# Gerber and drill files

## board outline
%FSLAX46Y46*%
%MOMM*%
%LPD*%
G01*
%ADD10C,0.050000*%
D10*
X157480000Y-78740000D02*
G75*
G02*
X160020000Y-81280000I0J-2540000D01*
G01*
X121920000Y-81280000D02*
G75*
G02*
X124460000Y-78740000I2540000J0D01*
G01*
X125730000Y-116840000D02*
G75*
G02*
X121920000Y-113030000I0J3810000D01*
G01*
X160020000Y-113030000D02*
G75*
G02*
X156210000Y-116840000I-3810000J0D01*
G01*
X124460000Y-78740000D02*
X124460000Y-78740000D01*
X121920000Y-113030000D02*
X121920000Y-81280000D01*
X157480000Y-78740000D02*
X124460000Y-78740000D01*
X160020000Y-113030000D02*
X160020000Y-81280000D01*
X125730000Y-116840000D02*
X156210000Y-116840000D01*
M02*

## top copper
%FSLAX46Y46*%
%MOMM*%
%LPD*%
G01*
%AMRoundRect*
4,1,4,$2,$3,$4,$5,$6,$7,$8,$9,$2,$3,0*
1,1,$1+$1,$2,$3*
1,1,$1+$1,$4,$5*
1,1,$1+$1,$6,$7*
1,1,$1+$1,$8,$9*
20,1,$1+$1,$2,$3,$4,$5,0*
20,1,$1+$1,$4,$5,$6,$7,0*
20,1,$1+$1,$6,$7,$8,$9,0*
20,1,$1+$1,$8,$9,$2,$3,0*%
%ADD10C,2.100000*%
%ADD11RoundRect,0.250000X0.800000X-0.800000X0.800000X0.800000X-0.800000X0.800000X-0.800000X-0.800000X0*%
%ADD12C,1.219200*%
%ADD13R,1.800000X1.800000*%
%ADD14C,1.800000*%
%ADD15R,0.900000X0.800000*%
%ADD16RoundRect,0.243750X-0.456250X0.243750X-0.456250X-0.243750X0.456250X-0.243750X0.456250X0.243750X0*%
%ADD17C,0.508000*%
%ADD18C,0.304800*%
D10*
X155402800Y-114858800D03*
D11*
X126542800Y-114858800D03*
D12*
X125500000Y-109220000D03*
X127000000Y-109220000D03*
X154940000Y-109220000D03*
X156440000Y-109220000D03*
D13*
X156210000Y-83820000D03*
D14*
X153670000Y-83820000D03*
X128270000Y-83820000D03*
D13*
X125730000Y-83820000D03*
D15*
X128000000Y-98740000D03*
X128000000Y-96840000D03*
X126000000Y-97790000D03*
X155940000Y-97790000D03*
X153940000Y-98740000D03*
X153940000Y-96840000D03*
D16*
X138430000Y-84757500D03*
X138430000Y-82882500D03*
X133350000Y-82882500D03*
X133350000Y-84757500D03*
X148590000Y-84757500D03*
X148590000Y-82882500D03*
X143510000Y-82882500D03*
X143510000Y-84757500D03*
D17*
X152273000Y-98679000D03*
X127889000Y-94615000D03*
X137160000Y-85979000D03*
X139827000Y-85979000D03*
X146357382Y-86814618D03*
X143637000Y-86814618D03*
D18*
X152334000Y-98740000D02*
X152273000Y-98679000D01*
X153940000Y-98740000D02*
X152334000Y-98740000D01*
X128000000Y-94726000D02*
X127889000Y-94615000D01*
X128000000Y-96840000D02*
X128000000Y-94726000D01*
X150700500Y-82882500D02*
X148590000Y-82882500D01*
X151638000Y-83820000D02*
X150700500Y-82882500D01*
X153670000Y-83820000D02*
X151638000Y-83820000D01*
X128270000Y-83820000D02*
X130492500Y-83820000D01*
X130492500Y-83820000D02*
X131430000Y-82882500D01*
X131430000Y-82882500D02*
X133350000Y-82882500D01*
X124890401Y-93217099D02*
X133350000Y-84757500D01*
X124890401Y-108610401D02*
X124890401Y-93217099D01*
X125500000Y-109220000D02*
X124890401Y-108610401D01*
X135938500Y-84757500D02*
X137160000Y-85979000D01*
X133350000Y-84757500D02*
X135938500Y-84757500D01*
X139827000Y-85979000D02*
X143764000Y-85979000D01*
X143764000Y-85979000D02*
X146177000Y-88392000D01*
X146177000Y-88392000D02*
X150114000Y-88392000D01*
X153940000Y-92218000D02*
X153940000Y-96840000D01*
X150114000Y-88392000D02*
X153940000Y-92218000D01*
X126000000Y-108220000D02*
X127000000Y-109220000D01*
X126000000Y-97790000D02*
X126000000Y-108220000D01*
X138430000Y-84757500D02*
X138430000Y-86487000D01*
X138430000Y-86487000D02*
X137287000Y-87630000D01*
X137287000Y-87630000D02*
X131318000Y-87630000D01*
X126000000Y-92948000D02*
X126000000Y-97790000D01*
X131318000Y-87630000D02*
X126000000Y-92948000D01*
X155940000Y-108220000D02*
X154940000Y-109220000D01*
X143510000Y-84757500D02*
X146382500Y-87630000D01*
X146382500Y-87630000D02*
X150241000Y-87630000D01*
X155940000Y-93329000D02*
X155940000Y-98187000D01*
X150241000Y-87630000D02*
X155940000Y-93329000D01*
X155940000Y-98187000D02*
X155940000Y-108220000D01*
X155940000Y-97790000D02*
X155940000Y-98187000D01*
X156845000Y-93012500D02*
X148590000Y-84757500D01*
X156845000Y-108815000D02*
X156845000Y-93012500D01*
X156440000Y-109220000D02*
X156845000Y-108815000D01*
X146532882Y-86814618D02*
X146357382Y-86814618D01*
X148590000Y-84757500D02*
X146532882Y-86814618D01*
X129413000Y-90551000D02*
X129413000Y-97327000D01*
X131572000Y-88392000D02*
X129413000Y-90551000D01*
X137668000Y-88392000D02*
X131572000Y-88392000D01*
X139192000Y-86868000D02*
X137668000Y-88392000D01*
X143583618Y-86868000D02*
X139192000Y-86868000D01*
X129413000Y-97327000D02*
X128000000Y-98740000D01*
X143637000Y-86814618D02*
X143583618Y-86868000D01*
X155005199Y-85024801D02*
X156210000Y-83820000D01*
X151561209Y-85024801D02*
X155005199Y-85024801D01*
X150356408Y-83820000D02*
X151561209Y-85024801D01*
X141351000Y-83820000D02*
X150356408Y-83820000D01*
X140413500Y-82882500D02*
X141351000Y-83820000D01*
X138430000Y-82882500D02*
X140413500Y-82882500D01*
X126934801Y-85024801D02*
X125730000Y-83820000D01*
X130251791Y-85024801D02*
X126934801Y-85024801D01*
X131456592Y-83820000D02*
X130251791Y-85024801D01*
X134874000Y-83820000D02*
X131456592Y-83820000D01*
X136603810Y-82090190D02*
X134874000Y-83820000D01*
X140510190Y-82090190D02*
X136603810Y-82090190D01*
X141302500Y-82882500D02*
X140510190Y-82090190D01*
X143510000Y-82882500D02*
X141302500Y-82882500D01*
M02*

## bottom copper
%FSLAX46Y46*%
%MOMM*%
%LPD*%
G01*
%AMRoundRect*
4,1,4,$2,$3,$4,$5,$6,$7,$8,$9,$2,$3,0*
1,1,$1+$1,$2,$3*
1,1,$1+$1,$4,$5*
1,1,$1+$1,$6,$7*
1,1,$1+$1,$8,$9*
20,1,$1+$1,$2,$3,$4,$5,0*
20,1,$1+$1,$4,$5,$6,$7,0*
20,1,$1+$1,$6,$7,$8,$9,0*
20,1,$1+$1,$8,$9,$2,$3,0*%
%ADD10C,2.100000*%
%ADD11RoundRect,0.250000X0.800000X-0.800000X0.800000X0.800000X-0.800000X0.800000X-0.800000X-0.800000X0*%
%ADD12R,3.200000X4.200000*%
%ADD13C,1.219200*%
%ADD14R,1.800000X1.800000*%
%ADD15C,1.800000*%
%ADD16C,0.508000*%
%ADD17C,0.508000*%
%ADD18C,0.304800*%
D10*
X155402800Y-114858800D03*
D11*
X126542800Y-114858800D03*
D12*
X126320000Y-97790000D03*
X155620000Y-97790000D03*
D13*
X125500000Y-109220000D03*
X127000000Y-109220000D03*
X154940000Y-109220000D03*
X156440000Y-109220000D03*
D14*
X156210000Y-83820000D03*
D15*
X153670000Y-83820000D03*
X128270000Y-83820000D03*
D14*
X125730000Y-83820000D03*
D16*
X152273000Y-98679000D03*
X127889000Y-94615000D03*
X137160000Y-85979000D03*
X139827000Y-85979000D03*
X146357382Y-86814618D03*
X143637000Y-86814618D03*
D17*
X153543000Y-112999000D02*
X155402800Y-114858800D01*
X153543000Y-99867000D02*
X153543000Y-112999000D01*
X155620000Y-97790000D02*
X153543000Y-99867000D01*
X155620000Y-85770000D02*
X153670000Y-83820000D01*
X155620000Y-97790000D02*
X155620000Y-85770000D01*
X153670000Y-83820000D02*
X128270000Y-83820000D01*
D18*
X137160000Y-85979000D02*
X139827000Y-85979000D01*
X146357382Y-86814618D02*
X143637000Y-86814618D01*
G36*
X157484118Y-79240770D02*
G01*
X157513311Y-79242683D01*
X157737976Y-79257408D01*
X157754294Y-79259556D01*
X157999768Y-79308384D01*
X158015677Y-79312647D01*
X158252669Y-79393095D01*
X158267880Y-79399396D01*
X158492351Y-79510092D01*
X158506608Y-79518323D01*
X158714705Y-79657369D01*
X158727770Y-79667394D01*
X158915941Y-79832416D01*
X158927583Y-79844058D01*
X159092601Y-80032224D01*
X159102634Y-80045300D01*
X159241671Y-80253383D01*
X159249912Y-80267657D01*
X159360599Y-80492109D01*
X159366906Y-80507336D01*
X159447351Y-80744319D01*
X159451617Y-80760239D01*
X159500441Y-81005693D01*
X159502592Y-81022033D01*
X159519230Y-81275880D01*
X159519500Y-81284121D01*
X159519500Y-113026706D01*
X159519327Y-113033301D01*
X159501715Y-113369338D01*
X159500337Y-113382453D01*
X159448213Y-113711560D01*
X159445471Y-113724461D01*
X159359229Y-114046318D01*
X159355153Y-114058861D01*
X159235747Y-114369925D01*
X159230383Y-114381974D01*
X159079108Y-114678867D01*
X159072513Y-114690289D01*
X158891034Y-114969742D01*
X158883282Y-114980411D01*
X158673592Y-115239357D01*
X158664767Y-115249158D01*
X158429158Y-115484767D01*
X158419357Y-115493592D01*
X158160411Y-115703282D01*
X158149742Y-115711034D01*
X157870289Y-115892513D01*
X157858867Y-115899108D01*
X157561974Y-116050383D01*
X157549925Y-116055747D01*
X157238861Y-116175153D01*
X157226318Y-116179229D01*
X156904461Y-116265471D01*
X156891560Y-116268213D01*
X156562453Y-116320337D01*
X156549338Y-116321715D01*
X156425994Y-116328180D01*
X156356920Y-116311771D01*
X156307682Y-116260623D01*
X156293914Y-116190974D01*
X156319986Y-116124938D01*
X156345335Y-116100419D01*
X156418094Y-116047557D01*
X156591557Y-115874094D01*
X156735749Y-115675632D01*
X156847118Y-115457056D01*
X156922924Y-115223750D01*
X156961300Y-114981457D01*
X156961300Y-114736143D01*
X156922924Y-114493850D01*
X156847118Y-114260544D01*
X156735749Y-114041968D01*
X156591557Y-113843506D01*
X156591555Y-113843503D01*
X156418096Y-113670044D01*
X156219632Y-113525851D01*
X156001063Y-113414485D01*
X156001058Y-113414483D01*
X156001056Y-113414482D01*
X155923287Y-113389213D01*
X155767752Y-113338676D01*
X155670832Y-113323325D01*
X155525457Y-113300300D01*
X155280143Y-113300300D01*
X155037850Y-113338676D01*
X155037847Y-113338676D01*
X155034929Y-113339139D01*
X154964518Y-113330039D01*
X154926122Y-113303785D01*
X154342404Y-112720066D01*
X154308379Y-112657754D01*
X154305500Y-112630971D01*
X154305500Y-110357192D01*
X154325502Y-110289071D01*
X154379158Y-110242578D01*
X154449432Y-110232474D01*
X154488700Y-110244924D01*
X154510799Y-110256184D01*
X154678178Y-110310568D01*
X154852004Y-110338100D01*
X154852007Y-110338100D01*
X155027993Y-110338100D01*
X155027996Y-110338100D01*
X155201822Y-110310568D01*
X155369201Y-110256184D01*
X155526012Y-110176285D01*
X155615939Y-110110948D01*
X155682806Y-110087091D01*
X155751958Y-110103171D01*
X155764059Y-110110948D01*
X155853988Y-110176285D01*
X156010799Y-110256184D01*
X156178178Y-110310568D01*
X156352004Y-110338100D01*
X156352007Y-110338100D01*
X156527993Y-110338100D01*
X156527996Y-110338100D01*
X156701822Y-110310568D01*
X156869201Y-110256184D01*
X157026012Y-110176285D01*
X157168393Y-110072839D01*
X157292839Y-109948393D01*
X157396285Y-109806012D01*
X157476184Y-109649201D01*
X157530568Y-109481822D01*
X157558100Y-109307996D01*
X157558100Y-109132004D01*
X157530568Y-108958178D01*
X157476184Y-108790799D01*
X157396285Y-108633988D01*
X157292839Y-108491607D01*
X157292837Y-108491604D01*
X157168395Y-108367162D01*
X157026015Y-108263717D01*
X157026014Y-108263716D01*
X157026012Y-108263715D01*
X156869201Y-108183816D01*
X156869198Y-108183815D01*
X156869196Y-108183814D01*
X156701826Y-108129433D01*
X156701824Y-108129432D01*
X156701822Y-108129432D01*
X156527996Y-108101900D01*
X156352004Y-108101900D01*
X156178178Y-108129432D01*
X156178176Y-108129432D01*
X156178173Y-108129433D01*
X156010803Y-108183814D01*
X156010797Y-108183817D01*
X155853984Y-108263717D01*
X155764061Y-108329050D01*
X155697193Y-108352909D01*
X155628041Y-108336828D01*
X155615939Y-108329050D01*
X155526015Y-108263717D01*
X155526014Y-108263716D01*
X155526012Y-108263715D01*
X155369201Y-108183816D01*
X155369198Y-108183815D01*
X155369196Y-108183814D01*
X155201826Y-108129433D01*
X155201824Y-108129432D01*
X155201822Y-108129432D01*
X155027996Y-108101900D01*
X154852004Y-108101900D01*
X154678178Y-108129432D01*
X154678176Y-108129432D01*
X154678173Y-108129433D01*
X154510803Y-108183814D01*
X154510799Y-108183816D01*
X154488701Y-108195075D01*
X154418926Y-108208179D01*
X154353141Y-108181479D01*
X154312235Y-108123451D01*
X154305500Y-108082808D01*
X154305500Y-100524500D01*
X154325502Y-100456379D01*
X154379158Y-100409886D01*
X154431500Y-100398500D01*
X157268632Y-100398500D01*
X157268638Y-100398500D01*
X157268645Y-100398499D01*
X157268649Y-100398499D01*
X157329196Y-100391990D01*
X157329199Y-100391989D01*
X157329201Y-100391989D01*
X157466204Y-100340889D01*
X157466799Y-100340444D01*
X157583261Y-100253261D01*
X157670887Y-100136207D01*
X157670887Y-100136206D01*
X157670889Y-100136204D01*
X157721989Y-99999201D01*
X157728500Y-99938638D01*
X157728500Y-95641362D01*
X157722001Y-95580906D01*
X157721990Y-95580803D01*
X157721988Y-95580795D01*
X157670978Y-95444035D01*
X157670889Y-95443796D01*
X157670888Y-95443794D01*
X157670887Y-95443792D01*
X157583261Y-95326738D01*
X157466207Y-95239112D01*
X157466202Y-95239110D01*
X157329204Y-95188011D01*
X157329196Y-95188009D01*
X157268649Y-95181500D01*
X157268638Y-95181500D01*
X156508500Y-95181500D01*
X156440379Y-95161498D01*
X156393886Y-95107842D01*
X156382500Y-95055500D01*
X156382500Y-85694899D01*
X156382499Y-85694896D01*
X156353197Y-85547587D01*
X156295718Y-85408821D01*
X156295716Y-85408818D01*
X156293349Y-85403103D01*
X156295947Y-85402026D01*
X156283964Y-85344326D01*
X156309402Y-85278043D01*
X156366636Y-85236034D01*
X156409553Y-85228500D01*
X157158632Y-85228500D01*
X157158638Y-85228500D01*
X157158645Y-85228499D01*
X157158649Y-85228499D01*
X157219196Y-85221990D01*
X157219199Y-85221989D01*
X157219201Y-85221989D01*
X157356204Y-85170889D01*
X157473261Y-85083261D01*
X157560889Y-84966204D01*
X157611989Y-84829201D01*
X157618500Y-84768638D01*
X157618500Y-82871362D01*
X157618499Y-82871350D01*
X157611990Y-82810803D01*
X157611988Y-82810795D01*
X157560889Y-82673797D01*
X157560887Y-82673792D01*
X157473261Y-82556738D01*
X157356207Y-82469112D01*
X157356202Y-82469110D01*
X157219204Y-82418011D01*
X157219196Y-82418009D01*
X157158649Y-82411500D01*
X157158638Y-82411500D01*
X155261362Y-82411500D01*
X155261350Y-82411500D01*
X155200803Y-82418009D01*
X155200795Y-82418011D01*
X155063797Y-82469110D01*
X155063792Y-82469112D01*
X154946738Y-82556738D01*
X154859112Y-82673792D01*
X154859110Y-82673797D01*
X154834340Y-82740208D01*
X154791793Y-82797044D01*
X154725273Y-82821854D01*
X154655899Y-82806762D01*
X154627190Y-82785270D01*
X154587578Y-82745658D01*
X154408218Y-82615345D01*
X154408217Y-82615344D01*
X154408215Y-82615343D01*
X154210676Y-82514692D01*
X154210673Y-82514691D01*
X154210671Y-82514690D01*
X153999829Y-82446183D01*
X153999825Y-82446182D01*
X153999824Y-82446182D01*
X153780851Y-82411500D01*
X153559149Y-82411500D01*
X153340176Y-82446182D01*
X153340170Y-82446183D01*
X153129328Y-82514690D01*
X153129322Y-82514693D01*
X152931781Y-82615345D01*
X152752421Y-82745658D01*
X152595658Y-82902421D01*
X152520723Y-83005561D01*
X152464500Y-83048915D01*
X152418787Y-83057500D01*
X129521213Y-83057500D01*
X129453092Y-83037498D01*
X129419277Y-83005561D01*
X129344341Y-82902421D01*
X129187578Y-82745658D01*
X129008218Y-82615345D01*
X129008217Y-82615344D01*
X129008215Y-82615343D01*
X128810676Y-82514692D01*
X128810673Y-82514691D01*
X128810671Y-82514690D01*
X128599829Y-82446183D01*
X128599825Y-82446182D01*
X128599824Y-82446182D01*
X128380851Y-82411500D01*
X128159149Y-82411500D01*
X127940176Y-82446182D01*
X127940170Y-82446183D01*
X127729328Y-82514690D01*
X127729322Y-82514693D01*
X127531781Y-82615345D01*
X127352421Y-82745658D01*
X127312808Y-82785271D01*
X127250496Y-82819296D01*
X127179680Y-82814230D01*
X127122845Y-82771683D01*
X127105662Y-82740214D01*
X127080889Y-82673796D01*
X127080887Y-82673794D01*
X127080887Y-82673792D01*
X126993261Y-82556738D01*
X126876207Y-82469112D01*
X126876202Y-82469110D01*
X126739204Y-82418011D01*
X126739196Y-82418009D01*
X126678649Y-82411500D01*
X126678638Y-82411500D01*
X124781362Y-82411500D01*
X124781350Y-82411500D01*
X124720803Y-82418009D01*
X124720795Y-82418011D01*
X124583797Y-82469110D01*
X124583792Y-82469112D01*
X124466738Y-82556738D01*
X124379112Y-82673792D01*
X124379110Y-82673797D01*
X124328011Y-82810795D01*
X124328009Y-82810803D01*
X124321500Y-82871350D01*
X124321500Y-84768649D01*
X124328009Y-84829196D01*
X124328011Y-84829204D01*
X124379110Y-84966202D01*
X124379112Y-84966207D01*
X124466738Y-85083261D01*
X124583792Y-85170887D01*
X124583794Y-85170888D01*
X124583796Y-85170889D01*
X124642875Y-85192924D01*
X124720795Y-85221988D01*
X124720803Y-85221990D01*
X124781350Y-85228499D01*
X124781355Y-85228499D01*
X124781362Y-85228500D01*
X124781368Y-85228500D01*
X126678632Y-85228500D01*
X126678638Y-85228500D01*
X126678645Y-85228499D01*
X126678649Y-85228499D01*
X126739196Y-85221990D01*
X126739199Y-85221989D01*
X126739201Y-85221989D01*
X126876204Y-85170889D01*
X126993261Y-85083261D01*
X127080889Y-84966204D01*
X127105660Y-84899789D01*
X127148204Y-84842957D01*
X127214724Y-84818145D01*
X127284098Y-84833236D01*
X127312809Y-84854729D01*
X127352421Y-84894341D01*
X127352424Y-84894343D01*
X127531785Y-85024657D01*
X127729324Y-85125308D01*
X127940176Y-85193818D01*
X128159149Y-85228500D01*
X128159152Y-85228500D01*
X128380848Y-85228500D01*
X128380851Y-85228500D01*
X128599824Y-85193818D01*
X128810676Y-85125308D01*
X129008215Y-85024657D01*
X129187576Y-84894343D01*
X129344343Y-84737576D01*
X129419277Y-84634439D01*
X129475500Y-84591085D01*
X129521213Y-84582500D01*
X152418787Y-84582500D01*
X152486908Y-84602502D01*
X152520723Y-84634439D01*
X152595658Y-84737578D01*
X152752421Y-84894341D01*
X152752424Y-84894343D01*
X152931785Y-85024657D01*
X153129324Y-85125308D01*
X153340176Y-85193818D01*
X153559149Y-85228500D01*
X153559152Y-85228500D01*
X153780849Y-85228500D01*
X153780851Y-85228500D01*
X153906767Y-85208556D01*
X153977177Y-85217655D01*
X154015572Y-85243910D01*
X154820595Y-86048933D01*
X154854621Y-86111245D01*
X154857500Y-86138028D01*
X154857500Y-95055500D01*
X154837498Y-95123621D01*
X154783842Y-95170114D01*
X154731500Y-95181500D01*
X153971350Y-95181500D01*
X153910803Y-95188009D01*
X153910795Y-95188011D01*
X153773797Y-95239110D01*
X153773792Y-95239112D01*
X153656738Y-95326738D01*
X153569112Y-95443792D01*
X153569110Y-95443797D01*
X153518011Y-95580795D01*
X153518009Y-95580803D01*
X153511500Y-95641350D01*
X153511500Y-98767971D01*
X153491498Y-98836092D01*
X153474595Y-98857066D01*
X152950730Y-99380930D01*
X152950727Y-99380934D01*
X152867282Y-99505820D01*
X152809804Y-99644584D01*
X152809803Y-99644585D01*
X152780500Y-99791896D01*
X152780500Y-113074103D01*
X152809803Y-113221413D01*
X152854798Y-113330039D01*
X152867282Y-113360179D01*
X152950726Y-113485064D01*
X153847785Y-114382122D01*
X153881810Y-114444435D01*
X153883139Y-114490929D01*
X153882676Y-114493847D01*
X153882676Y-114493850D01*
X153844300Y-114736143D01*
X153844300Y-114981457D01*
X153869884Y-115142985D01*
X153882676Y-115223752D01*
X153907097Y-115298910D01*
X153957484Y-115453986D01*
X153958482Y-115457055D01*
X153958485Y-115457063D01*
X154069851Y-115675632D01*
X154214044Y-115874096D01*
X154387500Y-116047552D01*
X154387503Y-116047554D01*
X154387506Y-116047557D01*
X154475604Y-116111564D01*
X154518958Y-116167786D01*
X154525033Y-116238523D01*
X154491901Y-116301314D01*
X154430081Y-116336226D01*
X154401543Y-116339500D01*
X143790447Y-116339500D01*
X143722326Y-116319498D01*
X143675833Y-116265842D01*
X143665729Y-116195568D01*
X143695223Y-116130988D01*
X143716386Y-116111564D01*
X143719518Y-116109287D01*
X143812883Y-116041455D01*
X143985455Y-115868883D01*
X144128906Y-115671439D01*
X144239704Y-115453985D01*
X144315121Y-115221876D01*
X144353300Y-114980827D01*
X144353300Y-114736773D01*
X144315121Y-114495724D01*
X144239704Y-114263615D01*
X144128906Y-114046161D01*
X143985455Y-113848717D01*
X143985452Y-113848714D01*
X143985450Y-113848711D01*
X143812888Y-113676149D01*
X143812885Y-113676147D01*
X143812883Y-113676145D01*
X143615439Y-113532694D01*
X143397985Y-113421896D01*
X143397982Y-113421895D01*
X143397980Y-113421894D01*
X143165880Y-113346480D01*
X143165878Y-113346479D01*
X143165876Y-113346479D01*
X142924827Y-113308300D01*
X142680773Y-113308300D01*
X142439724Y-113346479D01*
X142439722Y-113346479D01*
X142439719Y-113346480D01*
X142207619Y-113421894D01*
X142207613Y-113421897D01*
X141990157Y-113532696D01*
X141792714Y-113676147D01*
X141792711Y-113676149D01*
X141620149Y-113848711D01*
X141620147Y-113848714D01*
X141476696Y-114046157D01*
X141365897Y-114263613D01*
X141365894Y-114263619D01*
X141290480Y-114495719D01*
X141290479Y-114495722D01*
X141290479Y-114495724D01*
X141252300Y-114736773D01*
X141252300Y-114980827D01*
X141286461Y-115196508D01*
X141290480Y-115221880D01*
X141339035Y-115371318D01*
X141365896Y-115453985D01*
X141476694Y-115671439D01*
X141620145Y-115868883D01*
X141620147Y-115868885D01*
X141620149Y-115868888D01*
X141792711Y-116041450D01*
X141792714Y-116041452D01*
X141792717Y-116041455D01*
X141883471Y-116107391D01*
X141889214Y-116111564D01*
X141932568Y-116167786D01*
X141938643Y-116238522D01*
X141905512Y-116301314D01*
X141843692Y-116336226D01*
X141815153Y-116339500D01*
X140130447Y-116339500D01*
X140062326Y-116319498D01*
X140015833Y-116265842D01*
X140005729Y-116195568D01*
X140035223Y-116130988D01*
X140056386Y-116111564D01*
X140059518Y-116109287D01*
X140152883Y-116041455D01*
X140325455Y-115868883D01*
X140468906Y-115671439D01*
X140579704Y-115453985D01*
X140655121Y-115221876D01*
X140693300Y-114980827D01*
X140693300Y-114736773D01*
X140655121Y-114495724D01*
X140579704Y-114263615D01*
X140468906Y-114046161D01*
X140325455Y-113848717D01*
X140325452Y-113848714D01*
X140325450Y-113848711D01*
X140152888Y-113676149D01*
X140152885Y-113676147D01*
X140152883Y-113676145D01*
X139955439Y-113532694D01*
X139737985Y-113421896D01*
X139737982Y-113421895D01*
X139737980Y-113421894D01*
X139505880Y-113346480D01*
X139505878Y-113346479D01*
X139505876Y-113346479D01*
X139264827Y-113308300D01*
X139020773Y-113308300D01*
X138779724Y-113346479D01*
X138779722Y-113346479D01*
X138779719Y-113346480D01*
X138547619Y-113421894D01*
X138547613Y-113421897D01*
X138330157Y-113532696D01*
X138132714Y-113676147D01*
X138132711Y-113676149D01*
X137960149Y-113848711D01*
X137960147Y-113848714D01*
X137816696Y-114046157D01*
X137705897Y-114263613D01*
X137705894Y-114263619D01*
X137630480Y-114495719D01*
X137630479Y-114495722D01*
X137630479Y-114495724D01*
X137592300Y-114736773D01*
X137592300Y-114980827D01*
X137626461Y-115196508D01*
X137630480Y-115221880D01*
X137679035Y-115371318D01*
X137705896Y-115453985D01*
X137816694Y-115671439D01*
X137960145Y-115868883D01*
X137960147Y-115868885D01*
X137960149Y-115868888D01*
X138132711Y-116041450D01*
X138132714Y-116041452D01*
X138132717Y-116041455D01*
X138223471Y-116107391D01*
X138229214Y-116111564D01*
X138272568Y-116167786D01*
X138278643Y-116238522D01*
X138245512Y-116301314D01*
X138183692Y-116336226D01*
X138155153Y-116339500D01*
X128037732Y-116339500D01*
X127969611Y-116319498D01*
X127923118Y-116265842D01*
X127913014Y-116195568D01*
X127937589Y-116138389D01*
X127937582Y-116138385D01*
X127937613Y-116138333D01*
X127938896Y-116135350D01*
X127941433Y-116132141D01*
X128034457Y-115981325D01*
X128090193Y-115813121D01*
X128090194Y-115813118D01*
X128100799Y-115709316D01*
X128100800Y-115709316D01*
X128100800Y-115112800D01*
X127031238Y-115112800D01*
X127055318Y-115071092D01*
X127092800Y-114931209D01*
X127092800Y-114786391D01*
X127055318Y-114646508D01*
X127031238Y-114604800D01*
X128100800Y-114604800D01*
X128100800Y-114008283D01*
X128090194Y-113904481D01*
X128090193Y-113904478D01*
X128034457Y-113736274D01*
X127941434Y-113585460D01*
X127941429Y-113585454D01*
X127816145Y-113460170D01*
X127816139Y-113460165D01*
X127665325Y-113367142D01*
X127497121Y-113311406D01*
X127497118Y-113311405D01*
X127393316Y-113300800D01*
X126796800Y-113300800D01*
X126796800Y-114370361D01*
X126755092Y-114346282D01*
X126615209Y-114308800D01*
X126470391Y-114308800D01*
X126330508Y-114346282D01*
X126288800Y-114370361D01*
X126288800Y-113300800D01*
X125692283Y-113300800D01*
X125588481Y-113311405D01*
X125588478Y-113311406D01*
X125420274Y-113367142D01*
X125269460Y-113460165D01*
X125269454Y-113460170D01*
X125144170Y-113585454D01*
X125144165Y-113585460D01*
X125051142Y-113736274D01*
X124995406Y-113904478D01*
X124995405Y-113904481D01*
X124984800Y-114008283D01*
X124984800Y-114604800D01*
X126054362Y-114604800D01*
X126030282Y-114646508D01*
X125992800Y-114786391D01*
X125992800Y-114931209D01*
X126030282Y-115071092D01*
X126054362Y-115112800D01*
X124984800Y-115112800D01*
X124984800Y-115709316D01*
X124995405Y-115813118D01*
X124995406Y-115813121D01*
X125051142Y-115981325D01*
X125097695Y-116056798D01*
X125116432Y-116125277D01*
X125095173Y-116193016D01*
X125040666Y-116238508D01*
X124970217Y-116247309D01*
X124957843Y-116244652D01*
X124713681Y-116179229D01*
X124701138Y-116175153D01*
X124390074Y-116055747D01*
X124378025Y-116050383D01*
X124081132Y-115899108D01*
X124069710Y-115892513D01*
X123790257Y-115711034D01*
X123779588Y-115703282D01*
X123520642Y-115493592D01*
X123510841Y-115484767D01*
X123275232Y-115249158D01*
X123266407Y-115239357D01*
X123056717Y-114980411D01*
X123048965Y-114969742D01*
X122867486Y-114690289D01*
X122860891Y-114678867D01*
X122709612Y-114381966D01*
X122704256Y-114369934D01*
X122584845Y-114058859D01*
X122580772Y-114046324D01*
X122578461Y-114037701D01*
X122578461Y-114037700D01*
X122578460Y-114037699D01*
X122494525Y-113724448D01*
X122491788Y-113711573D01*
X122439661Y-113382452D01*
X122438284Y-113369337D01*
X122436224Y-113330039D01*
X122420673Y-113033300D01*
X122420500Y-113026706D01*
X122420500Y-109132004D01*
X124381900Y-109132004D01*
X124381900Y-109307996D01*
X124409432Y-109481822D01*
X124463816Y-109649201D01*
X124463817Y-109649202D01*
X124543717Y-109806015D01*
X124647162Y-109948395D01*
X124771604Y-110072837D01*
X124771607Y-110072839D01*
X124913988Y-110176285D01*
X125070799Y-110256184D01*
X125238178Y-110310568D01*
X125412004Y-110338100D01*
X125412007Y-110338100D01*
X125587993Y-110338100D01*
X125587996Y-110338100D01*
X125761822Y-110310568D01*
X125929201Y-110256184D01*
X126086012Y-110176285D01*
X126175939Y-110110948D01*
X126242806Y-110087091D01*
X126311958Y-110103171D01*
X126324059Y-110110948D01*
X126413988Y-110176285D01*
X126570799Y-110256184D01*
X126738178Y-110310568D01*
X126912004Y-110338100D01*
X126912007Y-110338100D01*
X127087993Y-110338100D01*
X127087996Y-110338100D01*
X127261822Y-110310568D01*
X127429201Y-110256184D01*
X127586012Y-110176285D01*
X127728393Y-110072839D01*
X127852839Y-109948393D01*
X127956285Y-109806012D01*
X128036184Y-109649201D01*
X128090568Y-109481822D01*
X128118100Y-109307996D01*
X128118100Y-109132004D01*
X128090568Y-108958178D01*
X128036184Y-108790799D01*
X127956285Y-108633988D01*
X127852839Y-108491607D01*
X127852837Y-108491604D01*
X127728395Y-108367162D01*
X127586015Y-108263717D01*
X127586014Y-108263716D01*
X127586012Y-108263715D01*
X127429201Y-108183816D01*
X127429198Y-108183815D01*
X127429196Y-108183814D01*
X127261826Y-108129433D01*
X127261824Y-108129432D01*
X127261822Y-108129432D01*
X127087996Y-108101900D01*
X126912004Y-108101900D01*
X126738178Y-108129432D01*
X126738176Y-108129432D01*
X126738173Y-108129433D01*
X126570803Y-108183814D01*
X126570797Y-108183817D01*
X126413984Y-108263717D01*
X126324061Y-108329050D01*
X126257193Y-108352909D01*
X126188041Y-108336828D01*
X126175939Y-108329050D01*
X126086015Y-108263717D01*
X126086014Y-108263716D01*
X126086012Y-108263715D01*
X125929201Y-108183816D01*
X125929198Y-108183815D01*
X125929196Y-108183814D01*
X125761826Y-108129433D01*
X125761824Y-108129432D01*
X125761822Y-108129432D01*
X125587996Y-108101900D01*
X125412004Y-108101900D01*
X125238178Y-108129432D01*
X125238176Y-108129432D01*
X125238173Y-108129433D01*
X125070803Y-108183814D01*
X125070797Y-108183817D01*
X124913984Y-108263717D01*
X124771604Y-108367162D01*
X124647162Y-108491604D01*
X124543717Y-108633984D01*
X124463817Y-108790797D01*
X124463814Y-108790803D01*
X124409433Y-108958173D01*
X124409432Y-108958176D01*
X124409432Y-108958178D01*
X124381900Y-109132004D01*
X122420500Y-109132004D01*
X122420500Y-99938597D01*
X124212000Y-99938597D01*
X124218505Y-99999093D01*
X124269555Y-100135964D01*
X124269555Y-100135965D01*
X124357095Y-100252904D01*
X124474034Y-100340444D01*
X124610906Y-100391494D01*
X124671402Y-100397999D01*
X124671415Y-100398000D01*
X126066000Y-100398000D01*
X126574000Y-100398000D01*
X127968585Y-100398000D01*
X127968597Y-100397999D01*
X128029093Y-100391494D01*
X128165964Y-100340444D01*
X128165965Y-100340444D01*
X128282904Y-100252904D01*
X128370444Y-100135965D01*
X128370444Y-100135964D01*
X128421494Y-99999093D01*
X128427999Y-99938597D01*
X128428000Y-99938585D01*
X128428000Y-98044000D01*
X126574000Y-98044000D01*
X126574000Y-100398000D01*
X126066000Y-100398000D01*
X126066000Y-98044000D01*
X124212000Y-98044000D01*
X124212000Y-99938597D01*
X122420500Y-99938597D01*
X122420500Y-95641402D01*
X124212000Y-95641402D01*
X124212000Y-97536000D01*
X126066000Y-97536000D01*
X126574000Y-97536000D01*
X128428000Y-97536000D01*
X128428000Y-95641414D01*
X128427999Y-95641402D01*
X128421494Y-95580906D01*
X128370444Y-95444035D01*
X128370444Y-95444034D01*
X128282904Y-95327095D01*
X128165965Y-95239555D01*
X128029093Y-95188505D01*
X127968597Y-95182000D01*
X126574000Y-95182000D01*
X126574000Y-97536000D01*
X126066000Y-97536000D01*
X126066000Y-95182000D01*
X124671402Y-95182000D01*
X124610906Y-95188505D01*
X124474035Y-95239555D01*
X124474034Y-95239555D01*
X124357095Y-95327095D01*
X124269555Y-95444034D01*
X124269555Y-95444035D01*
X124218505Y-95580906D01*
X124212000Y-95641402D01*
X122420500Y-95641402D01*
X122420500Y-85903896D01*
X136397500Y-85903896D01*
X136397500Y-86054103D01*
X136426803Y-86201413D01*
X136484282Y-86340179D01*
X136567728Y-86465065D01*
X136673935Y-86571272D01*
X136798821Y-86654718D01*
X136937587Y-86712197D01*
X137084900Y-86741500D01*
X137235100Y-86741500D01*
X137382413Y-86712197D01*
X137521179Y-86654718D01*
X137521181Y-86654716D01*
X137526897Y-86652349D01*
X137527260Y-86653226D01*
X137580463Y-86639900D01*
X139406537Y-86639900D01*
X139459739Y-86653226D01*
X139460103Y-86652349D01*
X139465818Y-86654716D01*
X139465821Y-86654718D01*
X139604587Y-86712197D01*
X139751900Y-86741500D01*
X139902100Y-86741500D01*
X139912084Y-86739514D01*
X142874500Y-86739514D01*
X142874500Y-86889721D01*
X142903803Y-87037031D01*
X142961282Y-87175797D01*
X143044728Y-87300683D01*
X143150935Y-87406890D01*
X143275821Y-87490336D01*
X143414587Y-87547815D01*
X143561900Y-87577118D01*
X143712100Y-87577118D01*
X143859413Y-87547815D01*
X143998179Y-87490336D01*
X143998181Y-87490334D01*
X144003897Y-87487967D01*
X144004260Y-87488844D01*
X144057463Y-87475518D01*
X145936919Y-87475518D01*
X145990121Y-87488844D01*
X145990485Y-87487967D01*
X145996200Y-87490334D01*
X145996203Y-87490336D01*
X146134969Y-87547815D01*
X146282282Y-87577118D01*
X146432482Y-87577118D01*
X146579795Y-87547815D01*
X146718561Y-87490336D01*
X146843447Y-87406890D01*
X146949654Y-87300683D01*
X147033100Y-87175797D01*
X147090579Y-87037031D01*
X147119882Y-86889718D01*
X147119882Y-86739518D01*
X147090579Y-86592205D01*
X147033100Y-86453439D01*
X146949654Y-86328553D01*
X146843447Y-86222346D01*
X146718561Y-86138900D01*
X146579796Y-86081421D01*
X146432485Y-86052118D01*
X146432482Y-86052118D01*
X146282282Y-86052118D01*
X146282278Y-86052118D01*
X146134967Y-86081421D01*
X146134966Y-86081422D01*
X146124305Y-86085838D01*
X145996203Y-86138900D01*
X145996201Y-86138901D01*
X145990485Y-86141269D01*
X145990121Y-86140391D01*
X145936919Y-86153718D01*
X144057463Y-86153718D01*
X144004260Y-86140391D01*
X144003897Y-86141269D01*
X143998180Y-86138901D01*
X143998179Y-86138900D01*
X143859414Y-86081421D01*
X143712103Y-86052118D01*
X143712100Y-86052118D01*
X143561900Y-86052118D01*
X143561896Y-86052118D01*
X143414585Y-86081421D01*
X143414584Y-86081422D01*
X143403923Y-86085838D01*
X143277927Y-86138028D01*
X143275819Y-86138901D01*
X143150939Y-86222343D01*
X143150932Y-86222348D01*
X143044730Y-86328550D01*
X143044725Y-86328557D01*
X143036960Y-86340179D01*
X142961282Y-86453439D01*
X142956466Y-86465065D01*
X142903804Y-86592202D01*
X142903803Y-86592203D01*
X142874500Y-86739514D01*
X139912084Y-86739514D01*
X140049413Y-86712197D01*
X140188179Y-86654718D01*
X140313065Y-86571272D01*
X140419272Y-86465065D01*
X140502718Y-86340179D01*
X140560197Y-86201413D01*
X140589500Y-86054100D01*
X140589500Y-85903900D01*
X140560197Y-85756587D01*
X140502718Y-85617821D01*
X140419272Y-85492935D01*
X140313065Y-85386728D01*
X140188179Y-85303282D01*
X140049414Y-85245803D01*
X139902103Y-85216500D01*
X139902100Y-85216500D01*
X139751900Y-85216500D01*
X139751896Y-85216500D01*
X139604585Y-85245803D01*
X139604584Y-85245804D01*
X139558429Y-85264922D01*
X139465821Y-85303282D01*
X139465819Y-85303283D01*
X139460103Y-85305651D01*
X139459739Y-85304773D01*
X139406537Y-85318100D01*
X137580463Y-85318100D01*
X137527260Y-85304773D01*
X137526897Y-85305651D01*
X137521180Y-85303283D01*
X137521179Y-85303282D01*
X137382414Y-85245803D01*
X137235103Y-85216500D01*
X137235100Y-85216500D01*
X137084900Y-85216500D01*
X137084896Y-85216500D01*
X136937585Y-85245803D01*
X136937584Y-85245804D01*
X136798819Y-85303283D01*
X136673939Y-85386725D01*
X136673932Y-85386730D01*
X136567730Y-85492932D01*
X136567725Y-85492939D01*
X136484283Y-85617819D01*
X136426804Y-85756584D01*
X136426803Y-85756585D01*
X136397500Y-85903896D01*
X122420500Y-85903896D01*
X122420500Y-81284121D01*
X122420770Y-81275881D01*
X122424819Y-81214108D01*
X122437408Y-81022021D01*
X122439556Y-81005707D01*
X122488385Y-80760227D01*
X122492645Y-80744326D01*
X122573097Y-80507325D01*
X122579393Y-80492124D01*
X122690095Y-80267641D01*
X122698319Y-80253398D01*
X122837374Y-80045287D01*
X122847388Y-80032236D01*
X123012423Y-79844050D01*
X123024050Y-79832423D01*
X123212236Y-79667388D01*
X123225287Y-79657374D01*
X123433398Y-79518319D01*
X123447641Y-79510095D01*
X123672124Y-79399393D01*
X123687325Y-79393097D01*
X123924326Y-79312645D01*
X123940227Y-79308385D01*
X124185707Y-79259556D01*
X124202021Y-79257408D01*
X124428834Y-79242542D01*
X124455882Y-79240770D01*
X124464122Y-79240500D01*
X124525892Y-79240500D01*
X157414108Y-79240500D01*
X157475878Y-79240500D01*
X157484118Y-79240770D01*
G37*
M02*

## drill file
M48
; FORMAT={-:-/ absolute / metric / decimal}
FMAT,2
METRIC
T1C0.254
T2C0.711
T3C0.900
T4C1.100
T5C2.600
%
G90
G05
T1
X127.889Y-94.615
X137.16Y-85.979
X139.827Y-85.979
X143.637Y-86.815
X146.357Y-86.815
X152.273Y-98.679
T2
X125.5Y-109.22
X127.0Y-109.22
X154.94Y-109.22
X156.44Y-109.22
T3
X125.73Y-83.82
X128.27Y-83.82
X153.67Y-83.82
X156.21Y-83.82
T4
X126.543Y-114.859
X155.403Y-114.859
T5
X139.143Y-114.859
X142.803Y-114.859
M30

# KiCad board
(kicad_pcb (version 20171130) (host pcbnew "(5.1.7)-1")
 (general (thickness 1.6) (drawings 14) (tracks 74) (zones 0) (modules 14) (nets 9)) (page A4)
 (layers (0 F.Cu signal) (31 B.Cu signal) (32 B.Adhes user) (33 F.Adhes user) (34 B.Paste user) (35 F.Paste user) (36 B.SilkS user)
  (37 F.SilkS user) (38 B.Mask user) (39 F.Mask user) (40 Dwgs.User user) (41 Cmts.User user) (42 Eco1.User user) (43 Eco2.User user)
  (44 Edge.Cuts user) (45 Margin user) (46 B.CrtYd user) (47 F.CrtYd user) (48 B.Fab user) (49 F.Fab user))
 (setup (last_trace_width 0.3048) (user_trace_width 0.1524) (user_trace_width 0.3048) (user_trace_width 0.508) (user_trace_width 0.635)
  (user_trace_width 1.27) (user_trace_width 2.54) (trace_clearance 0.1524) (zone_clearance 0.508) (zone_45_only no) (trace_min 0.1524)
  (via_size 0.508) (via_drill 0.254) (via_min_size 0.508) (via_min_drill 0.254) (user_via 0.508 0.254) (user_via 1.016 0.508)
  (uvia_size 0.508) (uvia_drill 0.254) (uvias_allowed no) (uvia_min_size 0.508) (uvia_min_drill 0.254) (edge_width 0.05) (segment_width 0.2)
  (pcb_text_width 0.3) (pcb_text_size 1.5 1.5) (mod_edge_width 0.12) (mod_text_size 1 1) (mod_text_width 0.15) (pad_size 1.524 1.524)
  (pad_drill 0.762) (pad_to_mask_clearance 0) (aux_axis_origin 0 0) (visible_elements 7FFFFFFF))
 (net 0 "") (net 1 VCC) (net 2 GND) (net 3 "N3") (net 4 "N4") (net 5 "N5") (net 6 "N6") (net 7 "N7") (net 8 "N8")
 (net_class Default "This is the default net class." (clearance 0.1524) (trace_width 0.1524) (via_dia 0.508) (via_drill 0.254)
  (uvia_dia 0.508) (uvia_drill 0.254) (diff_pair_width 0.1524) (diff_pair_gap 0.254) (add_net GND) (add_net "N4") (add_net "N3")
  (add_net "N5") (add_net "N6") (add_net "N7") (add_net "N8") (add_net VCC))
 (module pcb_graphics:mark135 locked (layer F.Cu) (at 140.97 99.06)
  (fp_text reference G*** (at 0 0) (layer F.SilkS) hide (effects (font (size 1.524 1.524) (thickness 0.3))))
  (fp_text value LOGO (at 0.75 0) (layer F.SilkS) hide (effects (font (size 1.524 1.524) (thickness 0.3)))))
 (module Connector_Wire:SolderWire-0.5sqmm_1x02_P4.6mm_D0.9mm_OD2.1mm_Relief (layer F.Cu) (at 140.5128 114.8588)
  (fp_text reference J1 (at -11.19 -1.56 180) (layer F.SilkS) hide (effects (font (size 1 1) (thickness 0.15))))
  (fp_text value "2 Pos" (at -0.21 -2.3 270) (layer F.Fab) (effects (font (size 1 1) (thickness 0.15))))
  (pad "" np_thru_hole circle (at 2.29 0 270) (size 2.6 2.6) (drill 2.6) (layers *.Cu *.Mask))
  (pad "" np_thru_hole circle (at -1.37 0 90) (size 2.6 2.6) (drill 2.6) (layers *.Cu *.Mask))
  (pad 2 thru_hole circle (at 14.89 0 270) (size 2.1 2.1) (drill 1.1) (layers *.Cu *.Mask) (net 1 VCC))
  (pad 1 thru_hole roundrect (at -13.97 0 90) (size 2.1 2.1) (drill 1.1) (layers *.Cu *.Mask) (roundrect_rratio 0.119047619047619)
   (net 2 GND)))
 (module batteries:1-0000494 (layer B.Cu) (at 140.97 97.79 180)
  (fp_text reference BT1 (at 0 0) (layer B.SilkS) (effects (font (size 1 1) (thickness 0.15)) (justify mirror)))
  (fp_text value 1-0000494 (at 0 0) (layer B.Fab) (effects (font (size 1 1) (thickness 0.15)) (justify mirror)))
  (pad 2 smd rect (at 14.65 0 180) (size 3.2 4.2) (layers B.Cu B.Paste B.Mask) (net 2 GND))
  (pad 1 smd rect (at -14.65 0 180) (size 3.2 4.2) (layers B.Cu B.Paste B.Mask) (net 1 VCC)))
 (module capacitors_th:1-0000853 (layer F.Cu) (at 127 109.22 180)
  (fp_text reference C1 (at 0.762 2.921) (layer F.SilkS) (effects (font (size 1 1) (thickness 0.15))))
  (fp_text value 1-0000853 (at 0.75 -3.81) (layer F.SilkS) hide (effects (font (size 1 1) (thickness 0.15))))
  (pad 2 thru_hole circle (at 1.5 0 180) (size 1.2192 1.2192) (drill 0.7112) (layers *.Cu *.Mask) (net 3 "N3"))
  (pad 1 thru_hole circle (at 0 0 180) (size 1.2192 1.2192) (drill 0.7112) (layers *.Cu *.Mask) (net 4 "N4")))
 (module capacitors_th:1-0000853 (layer F.Cu) (at 154.94 109.22)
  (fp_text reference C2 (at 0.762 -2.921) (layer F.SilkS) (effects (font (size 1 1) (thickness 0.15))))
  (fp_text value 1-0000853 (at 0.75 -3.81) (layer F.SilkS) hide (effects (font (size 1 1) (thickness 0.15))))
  (pad 1 thru_hole circle (at 0 0) (size 1.2192 1.2192) (drill 0.7112) (layers *.Cu *.Mask) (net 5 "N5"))
  (pad 2 thru_hole circle (at 1.5 0) (size 1.2192 1.2192) (drill 0.7112) (layers *.Cu *.Mask) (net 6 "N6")))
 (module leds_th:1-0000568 (layer F.Cu) (at 156.21 83.82 180)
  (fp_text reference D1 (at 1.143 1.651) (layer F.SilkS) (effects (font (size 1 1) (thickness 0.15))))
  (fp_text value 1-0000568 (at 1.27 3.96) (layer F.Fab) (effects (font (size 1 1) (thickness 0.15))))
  (pad 1 thru_hole rect (at 0 0 180) (size 1.8 1.8) (drill 0.9) (layers *.Cu *.Mask) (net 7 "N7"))
  (pad 2 thru_hole circle (at 2.54 0 180) (size 1.8 1.8) (drill 0.9) (layers *.Cu *.Mask) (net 1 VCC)))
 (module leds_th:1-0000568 (layer F.Cu) (at 125.73 83.82)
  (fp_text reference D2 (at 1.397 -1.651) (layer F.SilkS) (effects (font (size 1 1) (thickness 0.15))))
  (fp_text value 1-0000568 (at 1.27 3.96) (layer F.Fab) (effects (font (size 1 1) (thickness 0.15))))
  (pad 2 thru_hole circle (at 2.54 0) (size 1.8 1.8) (drill 0.9) (layers *.Cu *.Mask) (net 1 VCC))
  (pad 1 thru_hole rect (at 0 0) (size 1.8 1.8) (drill 0.9) (layers *.Cu *.Mask) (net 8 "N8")))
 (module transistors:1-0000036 (layer F.Cu) (at 127 97.79 180)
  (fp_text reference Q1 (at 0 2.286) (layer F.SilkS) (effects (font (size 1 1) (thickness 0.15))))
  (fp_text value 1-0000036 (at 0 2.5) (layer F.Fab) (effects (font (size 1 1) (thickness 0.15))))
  (pad 1 smd rect (at -1 -0.95 180) (size 0.9 0.8) (layers F.Cu F.Paste F.Mask) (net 6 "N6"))
  (pad 2 smd rect (at -1 0.95 180) (size 0.9 0.8) (layers F.Cu F.Paste F.Mask) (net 2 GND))
  (pad 3 smd rect (at 1 0 180) (size 0.9 0.8) (layers F.Cu F.Paste F.Mask) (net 4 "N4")))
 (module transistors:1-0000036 (layer F.Cu) (at 154.94 97.79)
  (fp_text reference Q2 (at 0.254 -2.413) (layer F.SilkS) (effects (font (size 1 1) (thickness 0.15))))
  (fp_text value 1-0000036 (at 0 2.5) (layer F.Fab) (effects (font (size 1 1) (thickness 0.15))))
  (pad 3 smd rect (at 1 0) (size 0.9 0.8) (layers F.Cu F.Paste F.Mask) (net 5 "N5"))
  (pad 2 smd rect (at -1 0.95) (size 0.9 0.8) (layers F.Cu F.Paste F.Mask) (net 2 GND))
  (pad 1 smd rect (at -1 -0.95) (size 0.9 0.8) (layers F.Cu F.Paste F.Mask) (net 3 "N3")))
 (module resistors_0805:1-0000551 (layer F.Cu) (at 138.43 83.82 270)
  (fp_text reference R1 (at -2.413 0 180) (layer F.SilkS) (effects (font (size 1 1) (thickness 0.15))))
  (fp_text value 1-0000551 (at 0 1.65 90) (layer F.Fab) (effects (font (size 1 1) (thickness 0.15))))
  (pad 2 smd roundrect (at 0.9375 0 270) (size 0.975 1.4) (layers F.Cu F.Paste F.Mask) (roundrect_rratio 0.25) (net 4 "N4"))
  (pad 1 smd roundrect (at -0.9375 0 270) (size 0.975 1.4) (layers F.Cu F.Paste F.Mask) (roundrect_rratio 0.25) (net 7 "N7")))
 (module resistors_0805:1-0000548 (layer F.Cu) (at 133.35 83.82 270)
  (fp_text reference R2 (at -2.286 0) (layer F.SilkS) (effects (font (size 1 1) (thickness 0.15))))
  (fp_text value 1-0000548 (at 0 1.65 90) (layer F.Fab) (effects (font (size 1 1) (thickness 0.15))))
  (pad 1 smd roundrect (at -0.9375 0 270) (size 0.975 1.4) (layers F.Cu F.Paste F.Mask) (roundrect_rratio 0.25) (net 1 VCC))
  (pad 2 smd roundrect (at 0.9375 0 270) (size 0.975 1.4) (layers F.Cu F.Paste F.Mask) (roundrect_rratio 0.25) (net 3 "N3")))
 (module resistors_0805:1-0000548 (layer F.Cu) (at 148.59 83.82 270)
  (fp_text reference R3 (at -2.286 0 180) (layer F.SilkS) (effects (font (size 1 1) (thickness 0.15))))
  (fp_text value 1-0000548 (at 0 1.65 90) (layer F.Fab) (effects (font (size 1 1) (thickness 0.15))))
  (pad 2 smd roundrect (at 0.9375 0 270) (size 0.975 1.4) (layers F.Cu F.Paste F.Mask) (roundrect_rratio 0.25) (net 6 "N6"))
  (pad 1 smd roundrect (at -0.9375 0 270) (size 0.975 1.4) (layers F.Cu F.Paste F.Mask) (roundrect_rratio 0.25) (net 1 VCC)))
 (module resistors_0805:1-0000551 (layer F.Cu) (at 143.51 83.82 270)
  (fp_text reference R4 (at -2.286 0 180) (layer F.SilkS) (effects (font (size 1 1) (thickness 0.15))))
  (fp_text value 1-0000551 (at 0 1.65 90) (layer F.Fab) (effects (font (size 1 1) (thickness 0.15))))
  (pad 1 smd roundrect (at -0.9375 0 270) (size 0.975 1.4) (layers F.Cu F.Paste F.Mask) (roundrect_rratio 0.25) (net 8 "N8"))
  (pad 2 smd roundrect (at 0.9375 0 270) (size 0.975 1.4) (layers F.Cu F.Paste F.Mask) (roundrect_rratio 0.25) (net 5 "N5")))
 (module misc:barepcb (layer F.Cu) (at 276.098 160.528)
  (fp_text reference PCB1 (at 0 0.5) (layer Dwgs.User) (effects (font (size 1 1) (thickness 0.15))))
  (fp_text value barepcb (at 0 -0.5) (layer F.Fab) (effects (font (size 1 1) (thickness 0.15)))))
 (gr_arc (start 157.48 81.28) (end 160.02 81.28) (angle -90) (layer Edge.Cuts) (width 0.05))
 (gr_arc (start 124.46 81.28) (end 124.46 78.74) (angle -90) (layer Edge.Cuts) (width 0.05))
 (gr_arc (start 125.73 113.03) (end 121.92 113.03) (angle -90) (layer Edge.Cuts) (width 0.05))
 (gr_arc (start 156.21 113.03) (end 156.21 116.84) (angle -90) (layer Edge.Cuts) (width 0.05))
 (gr_line (start 124.46 78.74) (end 124.46 78.74) (layer Edge.Cuts) (width 0.05))
 (gr_line (start 121.92 113.03) (end 121.92 81.28) (layer Edge.Cuts) (width 0.05))
 (gr_line (start 157.48 78.74) (end 124.46 78.74) (layer Edge.Cuts) (width 0.05))
 (gr_line (start 160.02 113.03) (end 160.02 81.28) (layer Edge.Cuts) (width 0.05))
 (gr_line (start 125.73 116.84) (end 156.21 116.84) (layer Edge.Cuts) (width 0.05))
 (via (at 152.273 98.679) (size 0.508) (drill 0.254) (layers F.Cu B.Cu) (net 2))
 (segment (start 152.334 98.74) (end 152.273 98.679) (width 0.3048) (layer F.Cu) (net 2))
 (segment (start 153.94 98.74) (end 152.334 98.74) (width 0.3048) (layer F.Cu) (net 2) (status 10))
 (via (at 127.889 94.615) (size 0.508) (drill 0.254) (layers F.Cu B.Cu) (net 2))
 (segment (start 128 94.726) (end 127.889 94.615) (width 0.3048) (layer F.Cu) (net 2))
 (segment (start 128 96.84) (end 128 94.726) (width 0.3048) (layer F.Cu) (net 2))
 (segment (start 153.543 112.999) (end 155.4028 114.8588) (width 0.508) (layer B.Cu) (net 1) (status 20))
 (segment (start 153.543 99.867) (end 153.543 112.999) (width 0.508) (layer B.Cu) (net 1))
 (segment (start 155.62 97.79) (end 153.543 99.867) (width 0.508) (layer B.Cu) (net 1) (status 10))
 (segment (start 155.62 85.77) (end 153.67 83.82) (width 0.508) (layer B.Cu) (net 1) (status 20))
 (segment (start 155.62 97.79) (end 155.62 85.77) (width 0.508) (layer B.Cu) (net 1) (status 10))
 (segment (start 153.67 83.82) (end 128.27 83.82) (width 0.508) (layer B.Cu) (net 1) (status 30))
 (segment (start 150.7005 82.8825) (end 148.59 82.8825) (width 0.3048) (layer F.Cu) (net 1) (status 20))
 (segment (start 151.638 83.82) (end 150.7005 82.8825) (width 0.3048) (layer F.Cu) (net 1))
 (segment (start 153.67 83.82) (end 151.638 83.82) (width 0.3048) (layer F.Cu) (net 1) (status 10))
 (segment (start 128.27 83.82) (end 130.4925 83.82) (width 0.3048) (layer F.Cu) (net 1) (status 10))
 (segment (start 130.4925 83.82) (end 131.43 82.8825) (width 0.3048) (layer F.Cu) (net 1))
 (segment (start 131.43 82.8825) (end 133.35 82.8825) (width 0.3048) (layer F.Cu) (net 1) (status 20))
 (segment (start 124.890401 93.217099) (end 133.35 84.7575) (width 0.3048) (layer F.Cu) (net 3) (status 20))
 (segment (start 124.890401 108.610401) (end 124.890401 93.217099) (width 0.3048) (layer F.Cu) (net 3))
 (segment (start 125.5 109.22) (end 124.890401 108.610401) (width 0.3048) (layer F.Cu) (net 3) (status 10))
 (via (at 137.16 85.979) (size 0.508) (drill 0.254) (layers F.Cu B.Cu) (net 3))
 (segment (start 135.9385 84.7575) (end 137.16 85.979) (width 0.3048) (layer F.Cu) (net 3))
 (segment (start 133.35 84.7575) (end 135.9385 84.7575) (width 0.3048) (layer F.Cu) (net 3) (status 10))
 (via (at 139.827 85.979) (size 0.508) (drill 0.254) (layers F.Cu B.Cu) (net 3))
 (segment (start 137.16 85.979) (end 139.827 85.979) (width 0.3048) (layer B.Cu) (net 3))
 (segment (start 139.827 85.979) (end 143.764 85.979) (width 0.3048) (layer F.Cu) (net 3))
 (segment (start 143.764 85.979) (end 146.177 88.392) (width 0.3048) (layer F.Cu) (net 3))
 (segment (start 146.177 88.392) (end 150.114 88.392) (width 0.3048) (layer F.Cu) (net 3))
 (segment (start 153.94 92.218) (end 153.94 96.84) (width 0.3048) (layer F.Cu) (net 3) (status 20))
 (segment (start 150.114 88.392) (end 153.94 92.218) (width 0.3048) (layer F.Cu) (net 3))
 (segment (start 126 108.22) (end 127 109.22) (width 0.3048) (layer F.Cu) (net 4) (status 20))
 (segment (start 126 97.79) (end 126 108.22) (width 0.3048) (layer F.Cu) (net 4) (status 10))
 (segment (start 138.43 84.7575) (end 138.43 86.487) (width 0.3048) (layer F.Cu) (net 4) (status 10))
 (segment (start 138.43 86.487) (end 137.287 87.63) (width 0.3048) (layer F.Cu) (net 4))
 (segment (start 137.287 87.63) (end 131.318 87.63) (width 0.3048) (layer F.Cu) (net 4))
 (segment (start 126 92.948) (end 126 97.79) (width 0.3048) (layer F.Cu) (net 4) (status 20))
 (segment (start 131.318 87.63) (end 126 92.948) (width 0.3048) (layer F.Cu) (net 4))
 (segment (start 155.94 108.22) (end 154.94 109.22) (width 0.3048) (layer F.Cu) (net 5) (status 20))
 (segment (start 143.51 84.7575) (end 146.3825 87.63) (width 0.3048) (layer F.Cu) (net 5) (status 10))
 (segment (start 146.3825 87.63) (end 150.241 87.63) (width 0.3048) (layer F.Cu) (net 5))
 (segment (start 155.94 93.329) (end 155.94 98.187) (width 0.3048) (layer F.Cu) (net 5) (status 20))
 (segment (start 150.241 87.63) (end 155.94 93.329) (width 0.3048) (layer F.Cu) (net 5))
 (segment (start 155.94 98.187) (end 155.94 108.22) (width 0.3048) (layer F.Cu) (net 5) (status 10))
 (segment (start 155.94 97.79) (end 155.94 98.187) (width 0.3048) (layer F.Cu) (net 5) (status 30))
 (segment (start 156.845 93.0125) (end 148.59 84.7575) (width 0.3048) (layer F.Cu) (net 6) (status 20))
 (segment (start 156.845 108.815) (end 156.845 93.0125) (width 0.3048) (layer F.Cu) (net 6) (status 10))
 (segment (start 156.44 109.22) (end 156.845 108.815) (width 0.3048) (layer F.Cu) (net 6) (status 30))
 (via (at 146.357382 86.814618) (size 0.508) (drill 0.254) (layers F.Cu B.Cu) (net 6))
 (segment (start 146.532882 86.814618) (end 146.357382 86.814618) (width 0.3048) (layer F.Cu) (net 6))
 (segment (start 148.59 84.7575) (end 146.532882 86.814618) (width 0.3048) (layer F.Cu) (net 6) (status 10))
 (segment (start 146.357382 86.814618) (end 143.637 86.814618) (width 0.3048) (layer B.Cu) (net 6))
 (via (at 143.637 86.814618) (size 0.508) (drill 0.254) (layers F.Cu B.Cu) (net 6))
 (segment (start 129.413 90.551) (end 129.413 97.327) (width 0.3048) (layer F.Cu) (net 6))
 (segment (start 131.572 88.392) (end 129.413 90.551) (width 0.3048) (layer F.Cu) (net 6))
 (segment (start 137.668 88.392) (end 131.572 88.392) (width 0.3048) (layer F.Cu) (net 6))
 (segment (start 139.192 86.868) (end 137.668 88.392) (width 0.3048) (layer F.Cu) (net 6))
 (segment (start 143.583618 86.868) (end 139.192 86.868) (width 0.3048) (layer F.Cu) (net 6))
 (segment (start 129.413 97.327) (end 128 98.74) (width 0.3048) (layer F.Cu) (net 6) (status 20))
 (segment (start 143.637 86.814618) (end 143.583618 86.868) (width 0.3048) (layer F.Cu) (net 6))
 (segment (start 155.005199 85.024801) (end 156.21 83.82) (width 0.3048) (layer F.Cu) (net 7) (status 20))
 (segment (start 151.561209 85.024801) (end 155.005199 85.024801) (width 0.3048) (layer F.Cu) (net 7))
 (segment (start 150.356408 83.82) (end 151.561209 85.024801) (width 0.3048) (layer F.Cu) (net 7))
 (segment (start 141.351 83.82) (end 150.356408 83.82) (width 0.3048) (layer F.Cu) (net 7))
 (segment (start 140.4135 82.8825) (end 141.351 83.82) (width 0.3048) (layer F.Cu) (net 7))
 (segment (start 138.43 82.8825) (end 140.4135 82.8825) (width 0.3048) (layer F.Cu) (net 7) (status 10))
 (segment (start 126.934801 85.024801) (end 125.73 83.82) (width 0.3048) (layer F.Cu) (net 8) (status 20))
 (segment (start 130.251791 85.024801) (end 126.934801 85.024801) (width 0.3048) (layer F.Cu) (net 8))
 (segment (start 131.456592 83.82) (end 130.251791 85.024801) (width 0.3048) (layer F.Cu) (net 8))
 (segment (start 134.874 83.82) (end 131.456592 83.82) (width 0.3048) (layer F.Cu) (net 8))
 (segment (start 136.60381 82.09019) (end 134.874 83.82) (width 0.3048) (layer F.Cu) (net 8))
 (segment (start 140.51019 82.09019) (end 136.60381 82.09019) (width 0.3048) (layer F.Cu) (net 8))
 (segment (start 141.3025 82.8825) (end 140.51019 82.09019) (width 0.3048) (layer F.Cu) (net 8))
 (segment (start 143.51 82.8825) (end 141.3025 82.8825) (width 0.3048) (layer F.Cu) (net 8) (status 10))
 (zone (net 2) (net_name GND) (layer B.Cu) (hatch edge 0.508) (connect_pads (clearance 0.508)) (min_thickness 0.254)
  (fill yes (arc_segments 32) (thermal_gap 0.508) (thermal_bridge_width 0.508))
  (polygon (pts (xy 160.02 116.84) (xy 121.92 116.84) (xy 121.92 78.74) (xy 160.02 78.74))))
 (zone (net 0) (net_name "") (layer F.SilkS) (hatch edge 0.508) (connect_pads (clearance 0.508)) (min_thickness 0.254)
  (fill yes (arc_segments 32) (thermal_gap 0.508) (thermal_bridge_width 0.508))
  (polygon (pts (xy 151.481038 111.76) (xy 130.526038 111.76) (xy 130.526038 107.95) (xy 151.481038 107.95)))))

